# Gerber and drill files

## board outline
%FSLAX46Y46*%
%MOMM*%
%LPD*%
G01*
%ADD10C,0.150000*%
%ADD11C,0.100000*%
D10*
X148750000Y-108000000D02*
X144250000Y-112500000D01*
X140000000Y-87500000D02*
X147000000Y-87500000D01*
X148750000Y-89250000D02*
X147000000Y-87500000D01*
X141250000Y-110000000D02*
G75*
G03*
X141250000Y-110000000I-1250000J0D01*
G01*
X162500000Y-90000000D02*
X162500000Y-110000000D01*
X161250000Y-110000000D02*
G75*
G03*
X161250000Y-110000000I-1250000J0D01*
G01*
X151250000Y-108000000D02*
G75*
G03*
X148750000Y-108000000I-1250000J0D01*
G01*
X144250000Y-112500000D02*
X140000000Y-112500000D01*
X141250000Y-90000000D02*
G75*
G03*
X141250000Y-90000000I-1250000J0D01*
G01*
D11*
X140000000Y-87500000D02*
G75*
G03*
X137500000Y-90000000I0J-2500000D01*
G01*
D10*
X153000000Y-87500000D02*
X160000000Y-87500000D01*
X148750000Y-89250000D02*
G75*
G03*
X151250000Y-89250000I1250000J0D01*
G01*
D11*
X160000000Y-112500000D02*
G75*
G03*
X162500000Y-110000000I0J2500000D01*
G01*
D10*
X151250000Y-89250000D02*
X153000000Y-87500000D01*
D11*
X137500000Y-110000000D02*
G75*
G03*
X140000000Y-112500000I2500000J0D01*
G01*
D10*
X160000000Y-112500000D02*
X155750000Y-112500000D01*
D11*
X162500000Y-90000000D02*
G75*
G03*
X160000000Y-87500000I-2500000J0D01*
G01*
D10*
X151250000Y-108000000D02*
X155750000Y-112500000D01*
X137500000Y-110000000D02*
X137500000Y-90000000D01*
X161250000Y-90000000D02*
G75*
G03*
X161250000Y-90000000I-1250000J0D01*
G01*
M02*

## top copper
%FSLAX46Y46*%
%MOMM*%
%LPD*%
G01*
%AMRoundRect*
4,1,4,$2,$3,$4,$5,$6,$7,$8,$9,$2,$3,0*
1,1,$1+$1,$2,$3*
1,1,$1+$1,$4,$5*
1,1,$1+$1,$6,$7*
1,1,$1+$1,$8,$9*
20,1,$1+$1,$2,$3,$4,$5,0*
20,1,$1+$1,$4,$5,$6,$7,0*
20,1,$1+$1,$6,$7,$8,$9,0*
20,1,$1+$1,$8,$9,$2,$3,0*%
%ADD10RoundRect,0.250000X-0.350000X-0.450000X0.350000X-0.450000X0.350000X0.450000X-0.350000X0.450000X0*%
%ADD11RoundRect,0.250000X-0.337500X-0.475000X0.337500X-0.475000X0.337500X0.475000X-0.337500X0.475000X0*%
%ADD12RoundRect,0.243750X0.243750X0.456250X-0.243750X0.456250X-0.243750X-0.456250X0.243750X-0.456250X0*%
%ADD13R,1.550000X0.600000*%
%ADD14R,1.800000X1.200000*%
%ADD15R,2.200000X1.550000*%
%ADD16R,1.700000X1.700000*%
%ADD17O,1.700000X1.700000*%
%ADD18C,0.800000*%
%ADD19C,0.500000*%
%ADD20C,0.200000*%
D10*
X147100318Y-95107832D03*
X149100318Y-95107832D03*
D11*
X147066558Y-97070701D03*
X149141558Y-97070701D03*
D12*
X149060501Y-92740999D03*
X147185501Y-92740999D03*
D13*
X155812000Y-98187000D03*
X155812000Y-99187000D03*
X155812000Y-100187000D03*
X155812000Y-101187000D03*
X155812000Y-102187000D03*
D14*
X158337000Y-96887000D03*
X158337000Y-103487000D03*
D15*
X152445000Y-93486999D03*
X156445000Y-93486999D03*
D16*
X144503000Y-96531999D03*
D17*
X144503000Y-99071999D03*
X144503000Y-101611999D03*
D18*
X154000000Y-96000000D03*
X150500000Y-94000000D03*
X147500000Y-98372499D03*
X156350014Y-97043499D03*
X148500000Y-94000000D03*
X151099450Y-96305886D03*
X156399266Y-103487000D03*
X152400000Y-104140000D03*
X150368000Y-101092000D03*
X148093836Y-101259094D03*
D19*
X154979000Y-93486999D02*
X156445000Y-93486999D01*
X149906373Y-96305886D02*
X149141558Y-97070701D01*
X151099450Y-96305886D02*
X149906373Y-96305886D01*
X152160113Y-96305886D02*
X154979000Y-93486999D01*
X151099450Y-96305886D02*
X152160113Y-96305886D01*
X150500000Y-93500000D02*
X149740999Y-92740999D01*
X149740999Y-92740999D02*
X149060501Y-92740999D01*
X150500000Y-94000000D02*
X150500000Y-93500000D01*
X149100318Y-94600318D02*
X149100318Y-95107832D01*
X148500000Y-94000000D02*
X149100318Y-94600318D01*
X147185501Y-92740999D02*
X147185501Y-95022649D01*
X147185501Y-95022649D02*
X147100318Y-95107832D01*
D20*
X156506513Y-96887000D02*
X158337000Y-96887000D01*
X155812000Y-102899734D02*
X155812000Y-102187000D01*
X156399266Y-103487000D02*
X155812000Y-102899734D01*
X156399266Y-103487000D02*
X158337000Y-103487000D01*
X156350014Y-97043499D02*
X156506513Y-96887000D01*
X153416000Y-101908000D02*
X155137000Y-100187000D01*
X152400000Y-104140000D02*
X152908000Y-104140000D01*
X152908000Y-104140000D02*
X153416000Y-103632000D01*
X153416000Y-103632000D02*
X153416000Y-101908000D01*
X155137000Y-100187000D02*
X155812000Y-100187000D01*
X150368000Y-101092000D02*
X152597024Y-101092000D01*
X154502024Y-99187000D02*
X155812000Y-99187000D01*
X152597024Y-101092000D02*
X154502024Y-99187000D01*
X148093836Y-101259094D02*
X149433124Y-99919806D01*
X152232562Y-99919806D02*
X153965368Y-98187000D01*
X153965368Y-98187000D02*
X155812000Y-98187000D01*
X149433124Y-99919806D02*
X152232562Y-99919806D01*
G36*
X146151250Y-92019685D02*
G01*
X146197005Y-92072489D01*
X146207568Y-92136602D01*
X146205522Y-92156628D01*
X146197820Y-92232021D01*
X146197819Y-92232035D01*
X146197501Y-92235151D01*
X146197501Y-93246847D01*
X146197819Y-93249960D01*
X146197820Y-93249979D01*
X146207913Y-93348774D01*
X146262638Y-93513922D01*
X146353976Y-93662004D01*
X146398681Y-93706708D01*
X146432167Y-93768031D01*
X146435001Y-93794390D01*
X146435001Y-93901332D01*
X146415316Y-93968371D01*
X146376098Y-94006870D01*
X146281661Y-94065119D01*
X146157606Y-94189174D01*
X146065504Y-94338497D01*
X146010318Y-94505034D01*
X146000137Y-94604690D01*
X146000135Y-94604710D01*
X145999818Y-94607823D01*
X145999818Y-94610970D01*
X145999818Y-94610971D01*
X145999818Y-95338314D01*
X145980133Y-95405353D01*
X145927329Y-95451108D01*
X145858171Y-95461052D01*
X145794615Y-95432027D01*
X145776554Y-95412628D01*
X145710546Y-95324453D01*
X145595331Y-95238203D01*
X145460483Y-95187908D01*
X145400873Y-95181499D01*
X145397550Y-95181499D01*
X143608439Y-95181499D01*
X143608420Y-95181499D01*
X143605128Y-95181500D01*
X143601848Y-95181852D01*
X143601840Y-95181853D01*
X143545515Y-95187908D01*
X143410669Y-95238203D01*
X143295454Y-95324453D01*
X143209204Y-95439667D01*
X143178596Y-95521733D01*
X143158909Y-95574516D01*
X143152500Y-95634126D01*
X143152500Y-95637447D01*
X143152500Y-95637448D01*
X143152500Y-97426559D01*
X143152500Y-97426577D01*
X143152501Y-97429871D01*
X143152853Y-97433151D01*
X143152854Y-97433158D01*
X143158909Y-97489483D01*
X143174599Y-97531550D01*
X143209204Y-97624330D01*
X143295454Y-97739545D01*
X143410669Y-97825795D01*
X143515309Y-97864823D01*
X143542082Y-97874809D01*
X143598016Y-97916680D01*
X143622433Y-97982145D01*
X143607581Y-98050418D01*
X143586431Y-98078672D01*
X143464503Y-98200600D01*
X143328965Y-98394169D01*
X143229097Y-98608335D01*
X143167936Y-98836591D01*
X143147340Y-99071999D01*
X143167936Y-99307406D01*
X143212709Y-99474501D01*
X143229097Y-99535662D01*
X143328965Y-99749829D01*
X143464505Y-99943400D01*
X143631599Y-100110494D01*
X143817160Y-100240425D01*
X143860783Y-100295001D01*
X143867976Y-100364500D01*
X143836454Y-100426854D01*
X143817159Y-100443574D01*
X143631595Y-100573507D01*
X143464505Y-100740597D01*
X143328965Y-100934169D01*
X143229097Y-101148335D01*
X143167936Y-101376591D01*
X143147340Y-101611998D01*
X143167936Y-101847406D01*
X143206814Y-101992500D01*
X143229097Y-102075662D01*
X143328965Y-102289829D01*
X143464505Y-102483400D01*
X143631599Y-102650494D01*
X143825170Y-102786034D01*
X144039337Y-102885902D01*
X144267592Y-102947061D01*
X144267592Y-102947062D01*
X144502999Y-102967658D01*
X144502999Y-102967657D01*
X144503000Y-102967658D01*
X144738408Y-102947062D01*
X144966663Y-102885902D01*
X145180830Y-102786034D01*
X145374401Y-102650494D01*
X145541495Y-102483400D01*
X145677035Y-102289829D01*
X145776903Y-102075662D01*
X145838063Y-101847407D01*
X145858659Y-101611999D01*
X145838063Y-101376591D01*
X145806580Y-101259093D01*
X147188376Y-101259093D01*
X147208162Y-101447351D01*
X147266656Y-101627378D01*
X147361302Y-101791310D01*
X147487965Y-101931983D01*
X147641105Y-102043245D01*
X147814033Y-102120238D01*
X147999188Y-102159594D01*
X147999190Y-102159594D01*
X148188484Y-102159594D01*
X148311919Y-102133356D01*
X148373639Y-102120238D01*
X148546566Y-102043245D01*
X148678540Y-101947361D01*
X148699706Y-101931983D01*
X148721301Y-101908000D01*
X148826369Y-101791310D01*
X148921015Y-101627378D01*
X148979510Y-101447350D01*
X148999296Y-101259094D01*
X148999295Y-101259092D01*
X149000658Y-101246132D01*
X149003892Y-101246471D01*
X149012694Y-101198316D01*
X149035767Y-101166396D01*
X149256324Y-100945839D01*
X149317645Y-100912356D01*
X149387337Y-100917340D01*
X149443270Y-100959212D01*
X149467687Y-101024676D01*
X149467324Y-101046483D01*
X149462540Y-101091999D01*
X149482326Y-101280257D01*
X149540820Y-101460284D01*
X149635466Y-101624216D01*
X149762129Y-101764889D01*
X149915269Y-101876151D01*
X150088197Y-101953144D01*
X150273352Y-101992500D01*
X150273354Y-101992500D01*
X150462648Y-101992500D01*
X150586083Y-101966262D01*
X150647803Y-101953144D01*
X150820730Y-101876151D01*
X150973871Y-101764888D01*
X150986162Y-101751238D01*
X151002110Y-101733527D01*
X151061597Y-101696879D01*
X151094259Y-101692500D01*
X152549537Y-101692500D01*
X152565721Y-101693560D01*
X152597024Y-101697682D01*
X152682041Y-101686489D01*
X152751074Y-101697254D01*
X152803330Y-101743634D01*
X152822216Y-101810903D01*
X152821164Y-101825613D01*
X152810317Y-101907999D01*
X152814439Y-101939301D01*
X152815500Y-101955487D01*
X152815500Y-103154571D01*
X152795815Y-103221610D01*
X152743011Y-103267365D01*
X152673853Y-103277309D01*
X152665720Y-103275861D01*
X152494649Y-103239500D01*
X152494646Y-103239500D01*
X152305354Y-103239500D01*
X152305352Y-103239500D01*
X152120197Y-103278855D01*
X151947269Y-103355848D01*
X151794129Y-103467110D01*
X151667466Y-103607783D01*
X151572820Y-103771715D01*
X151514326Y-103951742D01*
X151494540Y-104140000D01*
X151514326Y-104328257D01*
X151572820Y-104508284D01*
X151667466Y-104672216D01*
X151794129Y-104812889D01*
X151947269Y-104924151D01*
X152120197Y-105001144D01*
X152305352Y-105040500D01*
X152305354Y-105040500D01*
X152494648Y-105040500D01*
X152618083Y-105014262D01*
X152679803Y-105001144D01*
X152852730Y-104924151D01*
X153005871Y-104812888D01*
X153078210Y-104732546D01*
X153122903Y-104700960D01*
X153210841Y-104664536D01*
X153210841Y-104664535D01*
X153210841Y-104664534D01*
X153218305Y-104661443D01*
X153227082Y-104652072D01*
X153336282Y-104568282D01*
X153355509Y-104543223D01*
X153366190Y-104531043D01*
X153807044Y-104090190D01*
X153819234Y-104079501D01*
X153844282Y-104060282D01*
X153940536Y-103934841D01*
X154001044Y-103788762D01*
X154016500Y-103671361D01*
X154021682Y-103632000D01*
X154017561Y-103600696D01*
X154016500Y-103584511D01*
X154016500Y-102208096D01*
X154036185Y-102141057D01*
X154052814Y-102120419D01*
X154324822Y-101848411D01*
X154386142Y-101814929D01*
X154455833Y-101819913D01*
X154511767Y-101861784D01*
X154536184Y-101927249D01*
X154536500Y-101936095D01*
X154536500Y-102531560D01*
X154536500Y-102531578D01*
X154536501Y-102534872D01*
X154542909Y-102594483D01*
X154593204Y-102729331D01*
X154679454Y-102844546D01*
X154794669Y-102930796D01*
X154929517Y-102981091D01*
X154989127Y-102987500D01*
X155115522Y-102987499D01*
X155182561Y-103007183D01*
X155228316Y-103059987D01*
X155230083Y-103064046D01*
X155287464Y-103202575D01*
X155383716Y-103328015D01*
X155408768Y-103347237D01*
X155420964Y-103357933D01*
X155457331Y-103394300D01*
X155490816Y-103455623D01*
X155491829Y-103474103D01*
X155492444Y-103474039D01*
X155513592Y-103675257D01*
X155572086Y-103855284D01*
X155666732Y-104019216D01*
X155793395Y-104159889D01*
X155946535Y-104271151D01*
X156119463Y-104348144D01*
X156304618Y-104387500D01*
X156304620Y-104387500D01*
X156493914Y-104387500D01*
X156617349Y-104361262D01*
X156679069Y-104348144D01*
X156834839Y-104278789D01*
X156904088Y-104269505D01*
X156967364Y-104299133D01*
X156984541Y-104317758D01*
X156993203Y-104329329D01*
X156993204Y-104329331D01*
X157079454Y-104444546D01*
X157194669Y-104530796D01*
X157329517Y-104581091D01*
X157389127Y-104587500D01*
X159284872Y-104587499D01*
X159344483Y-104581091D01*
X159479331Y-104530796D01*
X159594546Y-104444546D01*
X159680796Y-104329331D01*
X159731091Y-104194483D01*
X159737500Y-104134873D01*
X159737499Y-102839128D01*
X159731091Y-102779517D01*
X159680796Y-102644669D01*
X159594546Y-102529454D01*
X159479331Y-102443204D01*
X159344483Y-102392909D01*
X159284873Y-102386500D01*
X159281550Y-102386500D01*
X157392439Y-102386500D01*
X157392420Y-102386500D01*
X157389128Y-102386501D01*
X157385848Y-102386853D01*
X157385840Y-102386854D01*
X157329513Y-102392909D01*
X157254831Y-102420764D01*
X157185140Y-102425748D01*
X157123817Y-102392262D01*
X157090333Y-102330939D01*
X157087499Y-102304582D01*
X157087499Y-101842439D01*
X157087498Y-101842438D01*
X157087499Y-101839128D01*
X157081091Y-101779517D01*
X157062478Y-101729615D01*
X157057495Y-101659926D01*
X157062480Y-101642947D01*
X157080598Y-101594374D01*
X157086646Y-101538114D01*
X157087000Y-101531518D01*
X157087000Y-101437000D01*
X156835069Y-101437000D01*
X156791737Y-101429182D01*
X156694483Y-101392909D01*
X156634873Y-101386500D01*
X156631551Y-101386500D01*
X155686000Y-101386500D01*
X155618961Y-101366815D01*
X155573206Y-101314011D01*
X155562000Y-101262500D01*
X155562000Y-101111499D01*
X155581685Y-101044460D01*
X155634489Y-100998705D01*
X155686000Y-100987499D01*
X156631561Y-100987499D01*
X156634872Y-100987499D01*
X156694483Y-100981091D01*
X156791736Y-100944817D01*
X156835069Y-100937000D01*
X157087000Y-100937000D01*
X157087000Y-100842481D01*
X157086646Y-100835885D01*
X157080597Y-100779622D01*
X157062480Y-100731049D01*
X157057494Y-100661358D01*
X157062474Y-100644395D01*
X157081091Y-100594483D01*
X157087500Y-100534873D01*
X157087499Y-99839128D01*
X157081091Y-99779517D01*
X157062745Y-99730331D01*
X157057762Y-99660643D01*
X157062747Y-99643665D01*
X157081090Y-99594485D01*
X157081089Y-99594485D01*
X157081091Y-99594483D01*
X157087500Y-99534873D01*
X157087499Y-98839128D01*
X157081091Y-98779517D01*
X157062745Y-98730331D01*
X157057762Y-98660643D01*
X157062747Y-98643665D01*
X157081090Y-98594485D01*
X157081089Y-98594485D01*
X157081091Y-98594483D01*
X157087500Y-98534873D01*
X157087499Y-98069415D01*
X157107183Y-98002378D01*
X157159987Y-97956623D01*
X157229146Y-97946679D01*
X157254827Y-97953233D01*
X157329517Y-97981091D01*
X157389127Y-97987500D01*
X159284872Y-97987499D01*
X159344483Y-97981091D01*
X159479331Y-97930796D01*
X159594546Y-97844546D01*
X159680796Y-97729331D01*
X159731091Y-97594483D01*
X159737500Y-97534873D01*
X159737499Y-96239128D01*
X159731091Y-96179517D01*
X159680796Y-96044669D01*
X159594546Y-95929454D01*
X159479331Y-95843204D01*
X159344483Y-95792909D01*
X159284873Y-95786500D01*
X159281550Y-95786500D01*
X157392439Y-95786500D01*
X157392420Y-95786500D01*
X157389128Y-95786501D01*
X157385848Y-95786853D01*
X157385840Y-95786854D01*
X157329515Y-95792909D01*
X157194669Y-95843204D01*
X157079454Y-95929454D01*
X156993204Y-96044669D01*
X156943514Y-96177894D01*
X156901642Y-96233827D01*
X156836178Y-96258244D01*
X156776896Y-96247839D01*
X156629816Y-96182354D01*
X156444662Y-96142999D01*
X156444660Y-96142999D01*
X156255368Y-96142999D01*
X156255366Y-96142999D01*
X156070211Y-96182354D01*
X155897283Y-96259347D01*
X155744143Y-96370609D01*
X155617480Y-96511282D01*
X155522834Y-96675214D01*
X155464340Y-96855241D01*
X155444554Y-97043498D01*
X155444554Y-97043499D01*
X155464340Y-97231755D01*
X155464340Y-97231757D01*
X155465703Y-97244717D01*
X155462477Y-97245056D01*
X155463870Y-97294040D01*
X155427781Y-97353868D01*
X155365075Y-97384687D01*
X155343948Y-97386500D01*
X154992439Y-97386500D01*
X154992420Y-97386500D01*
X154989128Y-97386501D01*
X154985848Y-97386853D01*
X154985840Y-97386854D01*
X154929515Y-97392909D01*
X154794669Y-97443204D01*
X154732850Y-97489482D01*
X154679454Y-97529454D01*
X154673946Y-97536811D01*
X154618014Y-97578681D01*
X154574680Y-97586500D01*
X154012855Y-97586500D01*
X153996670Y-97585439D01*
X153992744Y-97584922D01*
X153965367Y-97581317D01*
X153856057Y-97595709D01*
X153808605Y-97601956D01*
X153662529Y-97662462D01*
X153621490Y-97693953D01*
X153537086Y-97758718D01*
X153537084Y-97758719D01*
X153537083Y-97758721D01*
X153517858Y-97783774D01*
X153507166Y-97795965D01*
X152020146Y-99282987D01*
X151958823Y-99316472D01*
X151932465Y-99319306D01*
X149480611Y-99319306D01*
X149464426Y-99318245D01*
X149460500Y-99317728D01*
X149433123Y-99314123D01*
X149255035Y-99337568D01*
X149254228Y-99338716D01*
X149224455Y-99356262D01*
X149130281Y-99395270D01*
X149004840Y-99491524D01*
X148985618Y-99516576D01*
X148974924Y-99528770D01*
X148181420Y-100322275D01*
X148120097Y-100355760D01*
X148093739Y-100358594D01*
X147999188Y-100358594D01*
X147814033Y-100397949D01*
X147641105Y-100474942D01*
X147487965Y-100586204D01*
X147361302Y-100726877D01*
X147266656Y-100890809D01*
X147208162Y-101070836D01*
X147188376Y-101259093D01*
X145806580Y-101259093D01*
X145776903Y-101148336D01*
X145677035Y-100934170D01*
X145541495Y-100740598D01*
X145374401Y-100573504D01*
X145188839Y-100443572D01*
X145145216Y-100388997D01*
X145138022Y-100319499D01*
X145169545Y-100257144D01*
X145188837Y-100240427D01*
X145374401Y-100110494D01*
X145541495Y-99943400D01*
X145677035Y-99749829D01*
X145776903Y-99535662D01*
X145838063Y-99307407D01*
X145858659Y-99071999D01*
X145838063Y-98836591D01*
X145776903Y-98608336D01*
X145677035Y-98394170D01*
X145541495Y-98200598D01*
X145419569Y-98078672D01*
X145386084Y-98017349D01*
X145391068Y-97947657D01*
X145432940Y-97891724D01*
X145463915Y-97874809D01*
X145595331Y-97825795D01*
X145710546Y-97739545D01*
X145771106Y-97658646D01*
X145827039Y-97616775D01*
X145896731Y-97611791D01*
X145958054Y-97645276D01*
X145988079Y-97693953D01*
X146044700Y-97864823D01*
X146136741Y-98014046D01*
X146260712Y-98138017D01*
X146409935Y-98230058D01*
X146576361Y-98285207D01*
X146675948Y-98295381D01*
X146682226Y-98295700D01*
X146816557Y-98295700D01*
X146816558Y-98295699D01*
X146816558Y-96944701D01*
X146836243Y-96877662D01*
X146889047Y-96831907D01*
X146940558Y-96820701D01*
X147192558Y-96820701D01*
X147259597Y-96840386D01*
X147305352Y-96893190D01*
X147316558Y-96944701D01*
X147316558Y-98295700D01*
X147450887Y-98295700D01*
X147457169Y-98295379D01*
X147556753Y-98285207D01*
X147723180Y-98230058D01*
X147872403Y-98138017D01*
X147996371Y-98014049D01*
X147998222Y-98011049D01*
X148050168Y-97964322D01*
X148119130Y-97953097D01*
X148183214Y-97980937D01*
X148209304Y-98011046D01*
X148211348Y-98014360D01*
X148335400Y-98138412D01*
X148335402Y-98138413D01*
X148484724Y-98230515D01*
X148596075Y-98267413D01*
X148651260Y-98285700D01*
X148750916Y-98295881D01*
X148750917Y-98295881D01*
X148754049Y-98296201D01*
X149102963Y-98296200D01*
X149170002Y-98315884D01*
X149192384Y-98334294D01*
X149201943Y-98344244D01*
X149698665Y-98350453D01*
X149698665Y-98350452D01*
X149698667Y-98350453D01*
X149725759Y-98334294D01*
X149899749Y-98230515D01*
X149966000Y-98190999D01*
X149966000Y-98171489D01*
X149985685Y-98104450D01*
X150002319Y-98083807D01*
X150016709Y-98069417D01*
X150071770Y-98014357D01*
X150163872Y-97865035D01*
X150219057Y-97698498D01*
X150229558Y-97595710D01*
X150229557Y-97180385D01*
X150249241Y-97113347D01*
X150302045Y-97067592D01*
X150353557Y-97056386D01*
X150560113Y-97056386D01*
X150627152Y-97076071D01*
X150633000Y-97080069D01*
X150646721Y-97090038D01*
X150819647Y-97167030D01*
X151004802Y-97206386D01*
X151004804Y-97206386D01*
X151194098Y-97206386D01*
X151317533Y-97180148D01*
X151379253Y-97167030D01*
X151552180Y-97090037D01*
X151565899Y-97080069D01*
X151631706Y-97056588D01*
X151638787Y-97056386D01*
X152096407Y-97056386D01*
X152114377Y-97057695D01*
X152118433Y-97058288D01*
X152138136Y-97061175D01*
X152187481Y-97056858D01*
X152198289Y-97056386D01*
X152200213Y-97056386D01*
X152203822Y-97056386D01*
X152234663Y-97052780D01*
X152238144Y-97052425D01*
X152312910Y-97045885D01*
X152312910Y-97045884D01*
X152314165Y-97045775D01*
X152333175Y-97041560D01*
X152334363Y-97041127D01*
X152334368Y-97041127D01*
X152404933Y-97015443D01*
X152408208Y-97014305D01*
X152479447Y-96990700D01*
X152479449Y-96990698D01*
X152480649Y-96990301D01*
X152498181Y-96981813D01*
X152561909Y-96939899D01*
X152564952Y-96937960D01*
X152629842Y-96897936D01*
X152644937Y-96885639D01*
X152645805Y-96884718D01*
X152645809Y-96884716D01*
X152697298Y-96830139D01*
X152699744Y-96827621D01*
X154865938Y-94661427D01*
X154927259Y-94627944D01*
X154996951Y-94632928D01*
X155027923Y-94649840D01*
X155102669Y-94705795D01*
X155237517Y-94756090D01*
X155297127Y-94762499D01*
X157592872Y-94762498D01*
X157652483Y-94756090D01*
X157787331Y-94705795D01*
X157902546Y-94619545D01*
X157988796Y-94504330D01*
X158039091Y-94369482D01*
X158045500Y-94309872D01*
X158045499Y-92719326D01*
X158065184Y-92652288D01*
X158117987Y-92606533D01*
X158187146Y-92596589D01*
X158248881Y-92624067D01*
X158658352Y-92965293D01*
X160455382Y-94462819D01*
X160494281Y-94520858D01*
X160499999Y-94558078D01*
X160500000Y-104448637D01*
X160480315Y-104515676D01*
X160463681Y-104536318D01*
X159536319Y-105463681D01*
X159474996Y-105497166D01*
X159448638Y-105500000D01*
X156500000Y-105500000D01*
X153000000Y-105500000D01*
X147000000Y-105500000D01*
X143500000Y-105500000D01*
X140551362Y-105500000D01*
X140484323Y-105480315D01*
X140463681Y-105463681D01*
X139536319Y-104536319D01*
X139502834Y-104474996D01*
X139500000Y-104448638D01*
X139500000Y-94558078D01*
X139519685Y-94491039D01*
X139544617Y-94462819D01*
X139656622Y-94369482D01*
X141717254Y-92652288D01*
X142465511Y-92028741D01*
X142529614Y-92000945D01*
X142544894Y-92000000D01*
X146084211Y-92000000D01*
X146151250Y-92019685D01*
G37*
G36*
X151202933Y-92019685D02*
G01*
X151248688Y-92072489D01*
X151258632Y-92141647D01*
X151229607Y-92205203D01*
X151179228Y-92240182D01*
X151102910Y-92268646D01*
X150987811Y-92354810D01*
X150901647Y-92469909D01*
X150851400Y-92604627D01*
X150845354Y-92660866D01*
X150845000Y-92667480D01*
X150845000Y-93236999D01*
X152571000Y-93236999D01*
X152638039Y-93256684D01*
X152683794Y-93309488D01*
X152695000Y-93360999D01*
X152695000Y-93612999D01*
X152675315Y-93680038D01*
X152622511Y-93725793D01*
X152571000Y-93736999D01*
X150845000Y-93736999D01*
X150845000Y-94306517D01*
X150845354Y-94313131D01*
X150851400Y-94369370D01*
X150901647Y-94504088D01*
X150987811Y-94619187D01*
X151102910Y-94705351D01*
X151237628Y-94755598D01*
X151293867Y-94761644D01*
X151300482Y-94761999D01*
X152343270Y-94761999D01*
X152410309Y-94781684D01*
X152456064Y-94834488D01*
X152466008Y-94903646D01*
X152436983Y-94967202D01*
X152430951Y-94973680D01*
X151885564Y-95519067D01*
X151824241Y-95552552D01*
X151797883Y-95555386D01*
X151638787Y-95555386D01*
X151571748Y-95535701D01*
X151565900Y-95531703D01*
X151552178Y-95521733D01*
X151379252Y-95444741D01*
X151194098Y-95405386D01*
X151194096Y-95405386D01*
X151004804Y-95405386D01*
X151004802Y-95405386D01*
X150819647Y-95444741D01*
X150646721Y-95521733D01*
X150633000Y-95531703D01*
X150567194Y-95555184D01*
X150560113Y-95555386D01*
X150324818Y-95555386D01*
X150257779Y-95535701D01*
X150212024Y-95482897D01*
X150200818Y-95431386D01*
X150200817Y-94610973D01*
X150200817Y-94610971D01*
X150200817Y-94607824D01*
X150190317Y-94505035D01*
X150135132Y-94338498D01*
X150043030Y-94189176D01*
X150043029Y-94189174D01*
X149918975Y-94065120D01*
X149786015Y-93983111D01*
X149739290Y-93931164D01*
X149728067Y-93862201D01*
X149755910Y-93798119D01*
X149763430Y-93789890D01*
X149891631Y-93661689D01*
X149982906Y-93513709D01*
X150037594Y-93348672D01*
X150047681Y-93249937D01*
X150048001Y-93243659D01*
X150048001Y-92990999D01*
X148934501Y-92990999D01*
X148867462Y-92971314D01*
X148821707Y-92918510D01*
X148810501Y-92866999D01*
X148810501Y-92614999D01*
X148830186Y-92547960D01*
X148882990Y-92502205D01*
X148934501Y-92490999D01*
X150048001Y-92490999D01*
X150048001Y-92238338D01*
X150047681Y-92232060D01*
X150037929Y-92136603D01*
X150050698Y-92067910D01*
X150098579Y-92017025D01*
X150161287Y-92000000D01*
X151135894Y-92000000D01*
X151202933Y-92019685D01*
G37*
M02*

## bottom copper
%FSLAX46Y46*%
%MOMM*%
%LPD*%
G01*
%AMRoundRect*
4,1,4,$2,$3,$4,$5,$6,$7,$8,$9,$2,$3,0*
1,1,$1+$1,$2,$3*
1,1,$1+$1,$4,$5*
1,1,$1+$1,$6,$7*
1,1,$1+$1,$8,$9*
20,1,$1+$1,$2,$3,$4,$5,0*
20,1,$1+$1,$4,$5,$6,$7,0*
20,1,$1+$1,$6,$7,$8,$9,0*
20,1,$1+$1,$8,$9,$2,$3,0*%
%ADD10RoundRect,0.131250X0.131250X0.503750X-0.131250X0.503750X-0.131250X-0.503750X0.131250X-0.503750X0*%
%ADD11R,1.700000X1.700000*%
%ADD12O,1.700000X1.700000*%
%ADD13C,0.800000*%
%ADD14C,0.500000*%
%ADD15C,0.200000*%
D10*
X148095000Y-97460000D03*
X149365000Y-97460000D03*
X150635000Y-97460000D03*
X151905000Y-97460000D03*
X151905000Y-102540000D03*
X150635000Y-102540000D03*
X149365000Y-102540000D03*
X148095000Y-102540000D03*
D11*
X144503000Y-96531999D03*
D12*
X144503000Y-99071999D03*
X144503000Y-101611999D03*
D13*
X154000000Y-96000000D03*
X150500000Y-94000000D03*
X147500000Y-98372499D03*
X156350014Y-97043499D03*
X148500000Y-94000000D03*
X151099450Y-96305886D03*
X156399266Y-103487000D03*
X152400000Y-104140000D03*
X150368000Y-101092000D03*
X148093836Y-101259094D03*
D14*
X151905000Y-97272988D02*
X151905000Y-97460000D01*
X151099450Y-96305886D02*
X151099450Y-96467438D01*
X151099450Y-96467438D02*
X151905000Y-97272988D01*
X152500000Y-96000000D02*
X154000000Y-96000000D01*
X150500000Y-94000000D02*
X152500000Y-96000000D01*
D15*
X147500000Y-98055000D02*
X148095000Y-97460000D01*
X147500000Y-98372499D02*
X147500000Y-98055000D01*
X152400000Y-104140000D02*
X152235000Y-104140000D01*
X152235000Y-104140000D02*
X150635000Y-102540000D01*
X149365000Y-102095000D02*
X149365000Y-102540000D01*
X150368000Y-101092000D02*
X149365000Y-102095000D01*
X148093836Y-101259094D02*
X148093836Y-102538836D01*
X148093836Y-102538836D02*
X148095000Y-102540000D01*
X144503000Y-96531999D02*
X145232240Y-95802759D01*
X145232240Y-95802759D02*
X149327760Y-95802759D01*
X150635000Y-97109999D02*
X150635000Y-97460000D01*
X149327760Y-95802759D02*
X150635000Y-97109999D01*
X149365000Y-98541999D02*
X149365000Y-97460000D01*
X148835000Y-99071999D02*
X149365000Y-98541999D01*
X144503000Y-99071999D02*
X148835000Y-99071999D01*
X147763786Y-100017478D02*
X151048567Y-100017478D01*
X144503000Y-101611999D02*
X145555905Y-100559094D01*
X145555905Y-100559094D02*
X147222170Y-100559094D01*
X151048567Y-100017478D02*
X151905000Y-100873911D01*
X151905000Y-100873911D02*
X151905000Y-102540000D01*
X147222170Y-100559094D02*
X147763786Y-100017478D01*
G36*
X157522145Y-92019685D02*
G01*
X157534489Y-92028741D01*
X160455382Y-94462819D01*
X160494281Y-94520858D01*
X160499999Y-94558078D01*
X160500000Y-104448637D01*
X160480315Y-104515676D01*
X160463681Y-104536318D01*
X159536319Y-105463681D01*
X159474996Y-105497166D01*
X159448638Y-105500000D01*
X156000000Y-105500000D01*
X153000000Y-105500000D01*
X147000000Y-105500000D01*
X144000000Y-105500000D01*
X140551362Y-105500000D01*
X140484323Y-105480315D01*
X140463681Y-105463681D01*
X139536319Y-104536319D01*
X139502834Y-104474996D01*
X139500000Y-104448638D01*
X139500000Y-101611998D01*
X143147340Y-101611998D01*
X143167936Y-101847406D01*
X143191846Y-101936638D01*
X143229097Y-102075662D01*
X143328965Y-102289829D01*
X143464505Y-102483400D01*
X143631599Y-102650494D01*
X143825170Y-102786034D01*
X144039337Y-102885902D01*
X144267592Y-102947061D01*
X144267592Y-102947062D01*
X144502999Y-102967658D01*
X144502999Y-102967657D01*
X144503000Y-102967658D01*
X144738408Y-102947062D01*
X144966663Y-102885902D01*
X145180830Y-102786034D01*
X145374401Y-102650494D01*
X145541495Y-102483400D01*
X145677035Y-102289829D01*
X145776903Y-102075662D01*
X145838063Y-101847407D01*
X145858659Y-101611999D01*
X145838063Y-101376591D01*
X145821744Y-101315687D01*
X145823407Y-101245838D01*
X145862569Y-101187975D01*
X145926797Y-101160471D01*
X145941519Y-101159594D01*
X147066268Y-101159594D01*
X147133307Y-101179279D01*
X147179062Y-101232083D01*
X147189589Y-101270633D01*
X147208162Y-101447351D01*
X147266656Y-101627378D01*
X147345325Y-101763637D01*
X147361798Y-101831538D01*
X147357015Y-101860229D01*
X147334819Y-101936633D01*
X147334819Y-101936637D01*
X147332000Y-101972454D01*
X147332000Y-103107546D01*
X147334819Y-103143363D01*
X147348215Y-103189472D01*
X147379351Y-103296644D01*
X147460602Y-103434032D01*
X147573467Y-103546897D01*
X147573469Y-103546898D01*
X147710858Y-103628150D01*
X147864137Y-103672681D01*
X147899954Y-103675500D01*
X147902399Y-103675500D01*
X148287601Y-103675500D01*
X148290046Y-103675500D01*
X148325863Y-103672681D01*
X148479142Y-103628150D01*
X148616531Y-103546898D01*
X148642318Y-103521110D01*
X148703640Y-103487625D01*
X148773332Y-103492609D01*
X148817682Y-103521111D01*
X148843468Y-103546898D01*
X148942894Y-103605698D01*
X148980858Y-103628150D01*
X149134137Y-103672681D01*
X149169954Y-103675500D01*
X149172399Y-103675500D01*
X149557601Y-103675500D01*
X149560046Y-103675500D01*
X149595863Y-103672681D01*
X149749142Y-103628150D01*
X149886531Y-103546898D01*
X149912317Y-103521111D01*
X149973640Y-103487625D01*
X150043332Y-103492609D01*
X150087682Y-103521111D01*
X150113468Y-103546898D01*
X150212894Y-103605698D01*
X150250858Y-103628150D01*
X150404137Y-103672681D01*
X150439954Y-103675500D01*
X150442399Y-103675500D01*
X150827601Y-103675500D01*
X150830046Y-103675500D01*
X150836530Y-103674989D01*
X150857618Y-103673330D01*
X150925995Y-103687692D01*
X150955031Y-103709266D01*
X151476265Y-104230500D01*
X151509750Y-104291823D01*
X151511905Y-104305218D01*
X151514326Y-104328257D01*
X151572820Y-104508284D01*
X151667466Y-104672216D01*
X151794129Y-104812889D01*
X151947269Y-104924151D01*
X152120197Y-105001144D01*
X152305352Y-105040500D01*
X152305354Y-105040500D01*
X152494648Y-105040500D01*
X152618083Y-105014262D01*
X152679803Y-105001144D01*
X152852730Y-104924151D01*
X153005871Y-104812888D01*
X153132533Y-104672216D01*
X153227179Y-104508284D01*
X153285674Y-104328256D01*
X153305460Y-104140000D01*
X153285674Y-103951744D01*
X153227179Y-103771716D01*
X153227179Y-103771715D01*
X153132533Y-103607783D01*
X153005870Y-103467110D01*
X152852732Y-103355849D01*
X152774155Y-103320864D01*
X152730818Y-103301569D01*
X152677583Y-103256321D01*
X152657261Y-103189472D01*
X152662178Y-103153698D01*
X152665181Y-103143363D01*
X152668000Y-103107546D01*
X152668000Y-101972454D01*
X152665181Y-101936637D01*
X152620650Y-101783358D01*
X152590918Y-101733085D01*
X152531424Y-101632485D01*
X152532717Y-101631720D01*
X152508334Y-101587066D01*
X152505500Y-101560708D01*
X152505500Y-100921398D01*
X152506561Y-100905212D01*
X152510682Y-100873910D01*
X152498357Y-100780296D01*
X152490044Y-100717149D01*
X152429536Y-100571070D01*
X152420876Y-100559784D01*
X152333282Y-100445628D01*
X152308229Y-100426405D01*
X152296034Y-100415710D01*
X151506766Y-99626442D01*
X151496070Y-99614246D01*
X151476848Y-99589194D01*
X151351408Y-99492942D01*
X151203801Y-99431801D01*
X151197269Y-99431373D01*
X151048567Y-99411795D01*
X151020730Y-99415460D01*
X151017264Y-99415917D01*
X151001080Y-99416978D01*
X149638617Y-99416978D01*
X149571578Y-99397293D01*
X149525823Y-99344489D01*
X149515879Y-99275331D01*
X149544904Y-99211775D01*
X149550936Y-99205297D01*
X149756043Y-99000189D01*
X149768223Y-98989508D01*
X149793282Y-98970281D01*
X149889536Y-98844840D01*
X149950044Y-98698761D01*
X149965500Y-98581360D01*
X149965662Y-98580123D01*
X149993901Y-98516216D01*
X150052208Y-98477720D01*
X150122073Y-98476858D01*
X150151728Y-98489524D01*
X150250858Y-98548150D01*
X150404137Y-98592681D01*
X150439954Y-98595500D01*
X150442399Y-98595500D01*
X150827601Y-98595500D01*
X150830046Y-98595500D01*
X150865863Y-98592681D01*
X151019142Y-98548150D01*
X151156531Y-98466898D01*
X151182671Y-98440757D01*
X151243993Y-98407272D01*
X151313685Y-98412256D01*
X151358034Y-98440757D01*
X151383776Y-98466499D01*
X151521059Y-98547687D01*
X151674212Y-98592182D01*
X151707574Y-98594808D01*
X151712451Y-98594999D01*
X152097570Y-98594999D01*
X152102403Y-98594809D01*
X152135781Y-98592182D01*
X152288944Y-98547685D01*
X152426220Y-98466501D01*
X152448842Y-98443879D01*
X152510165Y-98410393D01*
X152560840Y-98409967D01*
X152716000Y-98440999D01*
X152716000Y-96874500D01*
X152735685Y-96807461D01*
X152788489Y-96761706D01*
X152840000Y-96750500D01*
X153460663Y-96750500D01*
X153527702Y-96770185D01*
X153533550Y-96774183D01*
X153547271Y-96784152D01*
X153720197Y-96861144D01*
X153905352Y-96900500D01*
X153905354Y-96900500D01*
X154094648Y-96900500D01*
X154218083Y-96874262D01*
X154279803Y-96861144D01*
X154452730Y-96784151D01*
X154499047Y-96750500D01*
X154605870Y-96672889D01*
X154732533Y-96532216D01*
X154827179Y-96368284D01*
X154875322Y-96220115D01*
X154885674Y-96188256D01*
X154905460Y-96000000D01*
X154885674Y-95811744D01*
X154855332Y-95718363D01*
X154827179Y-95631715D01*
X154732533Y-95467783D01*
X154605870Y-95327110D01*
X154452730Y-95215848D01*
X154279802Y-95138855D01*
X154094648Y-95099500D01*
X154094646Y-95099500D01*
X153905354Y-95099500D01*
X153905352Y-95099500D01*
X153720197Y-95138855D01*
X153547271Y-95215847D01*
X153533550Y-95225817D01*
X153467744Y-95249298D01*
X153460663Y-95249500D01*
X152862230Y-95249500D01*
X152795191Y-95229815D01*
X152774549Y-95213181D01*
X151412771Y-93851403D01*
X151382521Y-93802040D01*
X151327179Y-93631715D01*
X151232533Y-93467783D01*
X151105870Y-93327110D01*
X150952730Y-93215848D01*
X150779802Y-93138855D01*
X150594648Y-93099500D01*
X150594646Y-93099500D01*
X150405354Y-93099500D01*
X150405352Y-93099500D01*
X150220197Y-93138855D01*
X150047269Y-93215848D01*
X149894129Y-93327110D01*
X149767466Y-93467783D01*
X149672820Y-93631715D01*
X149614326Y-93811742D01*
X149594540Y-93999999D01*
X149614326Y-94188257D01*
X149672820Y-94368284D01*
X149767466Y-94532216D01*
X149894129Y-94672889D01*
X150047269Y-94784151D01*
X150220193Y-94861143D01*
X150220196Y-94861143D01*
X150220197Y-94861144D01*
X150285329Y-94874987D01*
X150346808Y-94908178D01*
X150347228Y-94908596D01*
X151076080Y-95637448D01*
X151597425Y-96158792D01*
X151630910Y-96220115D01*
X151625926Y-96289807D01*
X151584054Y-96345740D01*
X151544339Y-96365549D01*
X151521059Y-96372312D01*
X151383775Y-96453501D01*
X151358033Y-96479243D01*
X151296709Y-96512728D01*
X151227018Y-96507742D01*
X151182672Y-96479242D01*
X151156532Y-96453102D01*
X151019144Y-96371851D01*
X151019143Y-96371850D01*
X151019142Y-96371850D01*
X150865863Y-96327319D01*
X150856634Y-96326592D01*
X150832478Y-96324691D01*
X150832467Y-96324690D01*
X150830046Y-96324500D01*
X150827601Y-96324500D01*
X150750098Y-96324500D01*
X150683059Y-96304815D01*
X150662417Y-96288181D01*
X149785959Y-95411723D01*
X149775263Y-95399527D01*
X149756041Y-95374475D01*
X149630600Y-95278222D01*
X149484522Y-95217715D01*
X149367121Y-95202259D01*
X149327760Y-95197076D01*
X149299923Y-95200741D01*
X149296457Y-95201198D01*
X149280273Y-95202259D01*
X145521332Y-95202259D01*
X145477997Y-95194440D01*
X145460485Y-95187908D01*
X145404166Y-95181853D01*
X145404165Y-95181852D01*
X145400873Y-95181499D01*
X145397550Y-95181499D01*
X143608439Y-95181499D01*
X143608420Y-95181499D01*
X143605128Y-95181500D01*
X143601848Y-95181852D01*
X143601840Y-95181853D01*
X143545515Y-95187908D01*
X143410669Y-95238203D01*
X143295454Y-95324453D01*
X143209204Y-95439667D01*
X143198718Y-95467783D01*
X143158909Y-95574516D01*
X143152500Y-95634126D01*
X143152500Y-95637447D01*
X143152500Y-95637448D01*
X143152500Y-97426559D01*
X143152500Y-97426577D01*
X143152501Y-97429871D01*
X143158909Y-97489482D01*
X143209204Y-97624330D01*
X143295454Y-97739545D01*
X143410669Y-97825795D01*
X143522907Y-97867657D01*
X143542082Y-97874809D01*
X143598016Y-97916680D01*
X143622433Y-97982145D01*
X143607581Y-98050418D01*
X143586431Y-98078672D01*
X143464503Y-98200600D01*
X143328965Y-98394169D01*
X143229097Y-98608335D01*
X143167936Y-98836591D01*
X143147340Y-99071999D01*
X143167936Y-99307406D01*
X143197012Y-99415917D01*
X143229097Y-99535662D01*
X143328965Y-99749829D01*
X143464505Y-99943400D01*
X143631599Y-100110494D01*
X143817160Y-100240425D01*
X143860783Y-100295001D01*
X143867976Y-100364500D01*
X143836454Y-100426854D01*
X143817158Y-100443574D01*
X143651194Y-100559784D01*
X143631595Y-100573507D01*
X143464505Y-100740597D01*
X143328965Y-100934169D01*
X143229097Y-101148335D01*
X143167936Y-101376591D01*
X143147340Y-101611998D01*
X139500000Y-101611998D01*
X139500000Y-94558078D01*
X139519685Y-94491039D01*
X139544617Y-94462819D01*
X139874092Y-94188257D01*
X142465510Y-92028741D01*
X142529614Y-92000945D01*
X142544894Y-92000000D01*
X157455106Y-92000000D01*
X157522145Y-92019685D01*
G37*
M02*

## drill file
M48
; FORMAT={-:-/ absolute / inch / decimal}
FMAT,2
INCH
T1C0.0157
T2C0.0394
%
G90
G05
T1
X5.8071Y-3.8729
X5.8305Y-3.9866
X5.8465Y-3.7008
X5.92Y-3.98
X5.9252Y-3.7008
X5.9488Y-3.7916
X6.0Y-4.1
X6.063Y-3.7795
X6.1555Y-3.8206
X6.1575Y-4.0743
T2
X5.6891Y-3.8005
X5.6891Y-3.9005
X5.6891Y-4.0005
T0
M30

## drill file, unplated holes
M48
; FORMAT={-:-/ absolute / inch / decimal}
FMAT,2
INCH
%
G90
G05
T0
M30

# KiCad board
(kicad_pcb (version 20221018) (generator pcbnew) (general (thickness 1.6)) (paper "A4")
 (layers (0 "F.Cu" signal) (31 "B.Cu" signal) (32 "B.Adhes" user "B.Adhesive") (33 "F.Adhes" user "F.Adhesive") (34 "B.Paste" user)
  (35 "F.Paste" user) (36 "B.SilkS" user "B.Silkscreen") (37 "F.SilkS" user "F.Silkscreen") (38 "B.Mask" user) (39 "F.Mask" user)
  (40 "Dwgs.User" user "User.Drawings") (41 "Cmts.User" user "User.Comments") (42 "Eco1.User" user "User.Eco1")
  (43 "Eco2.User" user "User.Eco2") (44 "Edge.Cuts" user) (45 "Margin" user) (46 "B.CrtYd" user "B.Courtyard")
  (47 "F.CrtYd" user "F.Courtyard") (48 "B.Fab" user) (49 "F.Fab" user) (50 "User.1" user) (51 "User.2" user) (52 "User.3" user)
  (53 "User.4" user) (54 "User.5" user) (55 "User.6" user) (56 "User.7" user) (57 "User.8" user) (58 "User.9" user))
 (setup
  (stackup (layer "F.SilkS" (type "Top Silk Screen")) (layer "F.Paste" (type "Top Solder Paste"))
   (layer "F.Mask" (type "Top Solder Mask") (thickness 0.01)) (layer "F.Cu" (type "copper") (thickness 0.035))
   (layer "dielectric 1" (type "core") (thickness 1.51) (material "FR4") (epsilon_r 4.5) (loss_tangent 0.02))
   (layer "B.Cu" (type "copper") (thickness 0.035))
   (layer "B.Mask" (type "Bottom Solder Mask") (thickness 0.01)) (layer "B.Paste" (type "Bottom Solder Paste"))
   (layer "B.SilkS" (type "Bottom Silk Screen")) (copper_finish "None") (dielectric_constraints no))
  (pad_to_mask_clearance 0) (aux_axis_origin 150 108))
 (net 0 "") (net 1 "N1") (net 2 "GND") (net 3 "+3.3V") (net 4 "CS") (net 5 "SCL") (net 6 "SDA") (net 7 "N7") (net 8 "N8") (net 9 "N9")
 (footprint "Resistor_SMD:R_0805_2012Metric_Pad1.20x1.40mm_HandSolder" (layer "F.Cu") (at 148.100318 95.107832)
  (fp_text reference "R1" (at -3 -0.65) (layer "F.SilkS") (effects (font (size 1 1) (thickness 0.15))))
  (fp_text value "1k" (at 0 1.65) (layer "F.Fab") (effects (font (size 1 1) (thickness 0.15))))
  (pad "1" smd roundrect (at -1 0) (size 1.2 1.4) (layers "F.Cu" "F.Paste" "F.Mask") (roundrect_rratio 0.208333) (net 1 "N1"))
  (pad "2" smd roundrect (at 1 0) (size 1.2 1.4) (layers "F.Cu" "F.Paste" "F.Mask") (roundrect_rratio 0.208333) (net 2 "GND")))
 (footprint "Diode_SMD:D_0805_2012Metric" (layer "F.Cu") (at 148.123001 92.740999 180)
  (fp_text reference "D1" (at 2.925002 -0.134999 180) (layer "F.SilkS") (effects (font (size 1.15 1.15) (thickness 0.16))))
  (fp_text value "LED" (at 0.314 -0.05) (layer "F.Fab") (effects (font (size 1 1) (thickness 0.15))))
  (pad "1" smd roundrect (at -0.9375 0 180) (size 0.975 1.4) (layers "F.Cu" "F.Paste" "F.Mask") (roundrect_rratio 0.25) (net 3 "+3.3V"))
  (pad "2" smd roundrect (at 0.9375 0 180) (size 0.975 1.4) (layers "F.Cu" "F.Paste" "F.Mask") (roundrect_rratio 0.25) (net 1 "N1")))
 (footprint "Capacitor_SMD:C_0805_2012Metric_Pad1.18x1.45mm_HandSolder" (layer "F.Cu") (at 148.104058 97.070701)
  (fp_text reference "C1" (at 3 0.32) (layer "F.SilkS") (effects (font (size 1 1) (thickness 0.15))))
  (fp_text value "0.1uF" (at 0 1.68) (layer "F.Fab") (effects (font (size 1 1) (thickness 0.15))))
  (pad "1" smd roundrect (at -1.0375 0) (size 1.175 1.45) (layers "F.Cu" "F.Paste" "F.Mask") (roundrect_rratio 0.212766) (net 3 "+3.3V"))
  (pad "2" smd roundrect (at 1.0375 0) (size 1.175 1.45) (layers "F.Cu" "F.Paste" "F.Mask") (roundrect_rratio 0.212766) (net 2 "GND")))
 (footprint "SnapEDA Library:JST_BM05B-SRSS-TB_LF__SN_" (layer "F.Cu") (at 158.337 100.187 -90)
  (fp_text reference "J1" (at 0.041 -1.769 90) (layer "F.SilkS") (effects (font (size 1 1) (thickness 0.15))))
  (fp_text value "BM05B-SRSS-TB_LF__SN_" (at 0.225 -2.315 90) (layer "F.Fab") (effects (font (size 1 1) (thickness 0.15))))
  (pad "1" smd rect (at -2 2.525 270) (size 0.6 1.55) (layers "F.Cu" "F.Paste" "F.Mask") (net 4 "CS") (solder_mask_margin 0.102))
  (pad "2" smd rect (at -1 2.525 270) (size 0.6 1.55) (layers "F.Cu" "F.Paste" "F.Mask") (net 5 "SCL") (solder_mask_margin 0.102))
  (pad "3" smd rect (at 0 2.525 270) (size 0.6 1.55) (layers "F.Cu" "F.Paste" "F.Mask") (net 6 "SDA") (solder_mask_margin 0.102))
  (pad "4" smd rect (at 1 2.525 270) (size 0.6 1.55) (layers "F.Cu" "F.Paste" "F.Mask") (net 3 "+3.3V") (solder_mask_margin 0.102))
  (pad "5" smd rect (at 2 2.525 270) (size 0.6 1.55) (layers "F.Cu" "F.Paste" "F.Mask") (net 2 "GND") (solder_mask_margin 0.102))
  (pad "S1" smd rect (at -3.3 0 270) (size 1.2 1.8) (layers "F.Cu" "F.Paste" "F.Mask") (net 2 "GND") (solder_mask_margin 0.102))
  (pad "S2" smd rect (at 3.3 0 270) (size 1.2 1.8) (layers "F.Cu" "F.Paste" "F.Mask") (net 2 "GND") (solder_mask_margin 0.102)))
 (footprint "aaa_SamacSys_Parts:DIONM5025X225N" (layer "F.Cu") (at 154.445 93.486999)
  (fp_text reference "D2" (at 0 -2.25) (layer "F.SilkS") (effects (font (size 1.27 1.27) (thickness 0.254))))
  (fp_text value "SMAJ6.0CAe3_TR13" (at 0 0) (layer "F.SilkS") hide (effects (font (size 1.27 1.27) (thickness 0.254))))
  (pad "1" smd rect (at -2 0 90) (size 1.55 2.2) (layers "F.Cu" "F.Paste" "F.Mask") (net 3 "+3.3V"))
  (pad "2" smd rect (at 2 0 90) (size 1.55 2.2) (layers "F.Cu" "F.Paste" "F.Mask") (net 2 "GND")))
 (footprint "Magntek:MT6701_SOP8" (layer "B.Cu") (at 150 100)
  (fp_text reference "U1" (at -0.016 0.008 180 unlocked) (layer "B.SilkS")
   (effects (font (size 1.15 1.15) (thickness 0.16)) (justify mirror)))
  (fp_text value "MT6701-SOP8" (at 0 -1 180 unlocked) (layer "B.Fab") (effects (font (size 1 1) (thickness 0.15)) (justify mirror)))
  (pad "1" smd roundrect (at -1.905 -2.54 180) (size 0.525 1.27) (layers "B.Cu" "B.Paste" "B.Mask") (roundrect_rratio 0.25) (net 3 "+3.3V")
   (thermal_bridge_angle 45))
  (pad "2" smd roundrect (at -0.635 -2.54 180) (size 0.525 1.27) (layers "B.Cu" "B.Paste" "B.Mask") (roundrect_rratio 0.25) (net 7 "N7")
   (thermal_bridge_angle 45))
  (pad "3" smd roundrect (at 0.635 -2.54 180) (size 0.525 1.27) (layers "B.Cu" "B.Paste" "B.Mask") (roundrect_rratio 0.25) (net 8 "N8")
   (thermal_bridge_angle 45))
  (pad "4" smd roundrect (at 1.905 -2.54 180) (size 0.525 1.27) (layers "B.Cu" "B.Paste" "B.Mask") (roundrect_rratio 0.25) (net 2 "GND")
   (thermal_bridge_angle 45))
  (pad "5" smd roundrect (at 1.905 2.54 180) (size 0.525 1.27) (layers "B.Cu" "B.Paste" "B.Mask") (roundrect_rratio 0.25) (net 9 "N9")
   (thermal_bridge_angle 45))
  (pad "6" smd roundrect (at 0.635 2.54 180) (size 0.525 1.27) (layers "B.Cu" "B.Paste" "B.Mask") (roundrect_rratio 0.25) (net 6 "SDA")
   (thermal_bridge_angle 45))
  (pad "7" smd roundrect (at -0.635 2.54 180) (size 0.525 1.27) (layers "B.Cu" "B.Paste" "B.Mask") (roundrect_rratio 0.25) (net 5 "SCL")
   (thermal_bridge_angle 45))
  (pad "8" smd roundrect (at -1.905 2.54 180) (size 0.525 1.27) (layers "B.Cu" "B.Paste" "B.Mask") (roundrect_rratio 0.25) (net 4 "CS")
   (thermal_bridge_angle 45)))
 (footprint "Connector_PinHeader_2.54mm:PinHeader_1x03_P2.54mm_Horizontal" (layer "B.Cu") (at 144.503 96.531999 180)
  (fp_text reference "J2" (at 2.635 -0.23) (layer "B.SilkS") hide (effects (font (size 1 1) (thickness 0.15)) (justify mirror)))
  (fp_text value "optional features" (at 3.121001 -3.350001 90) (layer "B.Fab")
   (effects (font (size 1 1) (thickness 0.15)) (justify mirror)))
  (pad "1" thru_hole rect (at 0 0 180) (size 1.7 1.7) (drill 1) (layers "*.Cu" "*.Mask") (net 8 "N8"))
  (pad "2" thru_hole oval (at 0 -2.54 180) (size 1.7 1.7) (drill 1) (layers "*.Cu" "*.Mask") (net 7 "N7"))
  (pad "3" thru_hole oval (at 0 -5.08 180) (size 1.7 1.7) (drill 1) (layers "*.Cu" "*.Mask") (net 9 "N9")))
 (gr_line (start 148.75 108) (end 144.25 112.5) (stroke (width 0.15) (type default)) (layer "Edge.Cuts"))
 (gr_line (start 140 87.5) (end 147 87.5) (stroke (width 0.15) (type default)) (layer "Edge.Cuts"))
 (gr_line (start 148.75 89.25) (end 147 87.5) (stroke (width 0.15) (type default)) (layer "Edge.Cuts"))
 (gr_circle (center 140 110) (end 141.25 110) (stroke (width 0.15) (type default)) (fill none) (layer "Edge.Cuts"))
 (gr_line (start 162.5 90) (end 162.5 110) (stroke (width 0.15) (type default)) (layer "Edge.Cuts"))
 (gr_circle (center 160 110) (end 161.25 110) (stroke (width 0.15) (type default)) (fill none) (layer "Edge.Cuts"))
 (gr_arc (start 148.75 108) (mid 150 106.75) (end 151.25 108) (stroke (width 0.15) (type default)) (layer "Edge.Cuts"))
 (gr_line (start 144.25 112.5) (end 140 112.5) (stroke (width 0.15) (type default)) (layer "Edge.Cuts"))
 (gr_circle (center 140 90) (end 141.25 90) (stroke (width 0.15) (type default)) (fill none) (layer "Edge.Cuts"))
 (gr_arc (start 137.5 90) (mid 138.232233 88.232233) (end 140 87.5) (stroke (width 0.1) (type default)) (layer "Edge.Cuts"))
 (gr_line (start 153 87.5) (end 160 87.5) (stroke (width 0.15) (type default)) (layer "Edge.Cuts"))
 (gr_arc (start 151.25 89.25) (mid 150 90.5) (end 148.75 89.25) (stroke (width 0.15) (type default)) (layer "Edge.Cuts"))
 (gr_arc (start 162.5 110) (mid 161.767767 111.767767) (end 160 112.5) (stroke (width 0.1) (type default)) (layer "Edge.Cuts"))
 (gr_line (start 151.25 89.25) (end 153 87.5) (stroke (width 0.15) (type default)) (layer "Edge.Cuts"))
 (gr_arc (start 140 112.5) (mid 138.232233 111.767767) (end 137.5 110) (stroke (width 0.1) (type default)) (layer "Edge.Cuts"))
 (gr_line (start 160 112.5) (end 155.75 112.5) (stroke (width 0.15) (type default)) (layer "Edge.Cuts"))
 (gr_arc (start 160 87.5) (mid 161.767767 88.232233) (end 162.5 90) (stroke (width 0.1) (type default)) (layer "Edge.Cuts"))
 (gr_line (start 151.25 108) (end 155.75 112.5) (stroke (width 0.15) (type default)) (layer "Edge.Cuts"))
 (gr_line (start 137.5 110) (end 137.5 90) (stroke (width 0.15) (type default)) (layer "Edge.Cuts"))
 (gr_circle (center 160 90) (end 161.25 90) (stroke (width 0.15) (type default)) (fill none) (layer "Edge.Cuts"))
 (segment (start 150.5 93.5) (end 149.740999 92.740999) (width 0.5) (layer "F.Cu") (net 3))
 (segment (start 149.740999 92.740999) (end 149.060501 92.740999) (width 0.5) (layer "F.Cu") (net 3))
 (segment (start 150.5 94) (end 150.5 93.5) (width 0.5) (layer "F.Cu") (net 3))
 (via (at 150.5 94) (size 0.8) (drill 0.4) (layers "F.Cu" "B.Cu") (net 3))
 (via (at 147.5 98.372499) (size 0.8) (drill 0.4) (layers "F.Cu" "B.Cu") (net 3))
 (via (at 154 96) (size 0.8) (drill 0.4) (layers "F.Cu" "B.Cu") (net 3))
 (segment (start 147.5 98.055) (end 148.095 97.46) (width 0.2) (layer "B.Cu") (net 3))
 (segment (start 150.5 94) (end 152.5 96) (width 0.5) (layer "B.Cu") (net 3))
 (segment (start 147.5 98.372499) (end 147.5 98.055) (width 0.2) (layer "B.Cu") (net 3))
 (segment (start 152.5 96) (end 154 96) (width 0.5) (layer "B.Cu") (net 3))
 (segment (start 148.5 94) (end 149.100318 94.600318) (width 0.5) (layer "F.Cu") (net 2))
 (segment (start 156.506513 96.887) (end 158.337 96.887) (width 0.2) (layer "F.Cu") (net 2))
 (segment (start 155.812 102.899734) (end 155.812 102.187) (width 0.2) (layer "F.Cu") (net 2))
 (segment (start 156.399266 103.487) (end 155.812 102.899734) (width 0.2) (layer "F.Cu") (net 2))
 (segment (start 149.100318 94.600318) (end 149.100318 95.107832) (width 0.5) (layer "F.Cu") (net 2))
 (segment (start 151.09945 96.305886) (end 149.906373 96.305886) (width 0.5) (layer "F.Cu") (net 2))
 (segment (start 151.09945 96.305886) (end 152.160113 96.305886) (width 0.5) (layer "F.Cu") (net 2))
 (segment (start 149.906373 96.305886) (end 149.141558 97.070701) (width 0.5) (layer "F.Cu") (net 2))
 (segment (start 156.399266 103.487) (end 158.337 103.487) (width 0.2) (layer "F.Cu") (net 2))
 (segment (start 152.160113 96.305886) (end 154.979 93.486999) (width 0.5) (layer "F.Cu") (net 2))
 (segment (start 156.350014 97.043499) (end 156.506513 96.887) (width 0.2) (layer "F.Cu") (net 2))
 (segment (start 154.979 93.486999) (end 156.445 93.486999) (width 0.5) (layer "F.Cu") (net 2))
 (via (at 156.350014 97.043499) (size 0.8) (drill 0.4) (layers "F.Cu" "B.Cu") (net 2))
 (via (at 148.5 94) (size 0.8) (drill 0.4) (layers "F.Cu" "B.Cu") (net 2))
 (via (at 151.09945 96.305886) (size 0.8) (drill 0.4) (layers "F.Cu" "B.Cu") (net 2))
 (via (at 156.399266 103.487) (size 0.8) (drill 0.4) (layers "F.Cu" "B.Cu") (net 2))
 (segment (start 151.905 97.272988) (end 151.905 97.46) (width 0.5) (layer "B.Cu") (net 2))
 (segment (start 151.09945 96.467438) (end 151.905 97.272988) (width 0.5) (layer "B.Cu") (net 2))
 (segment (start 151.09945 96.305886) (end 151.09945 96.467438) (width 0.5) (layer "B.Cu") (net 2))
 (segment (start 147.185501 95.022649) (end 147.100318 95.107832) (width 0.5) (layer "F.Cu") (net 1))
 (segment (start 147.185501 92.740999) (end 147.185501 95.022649) (width 0.5) (layer "F.Cu") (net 1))
 (segment (start 153.416 101.908) (end 155.137 100.187) (width 0.2) (layer "F.Cu") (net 6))
 (segment (start 152.4 104.14) (end 152.908 104.14) (width 0.2) (layer "F.Cu") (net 6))
 (segment (start 152.908 104.14) (end 153.416 103.632) (width 0.2) (layer "F.Cu") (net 6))
 (segment (start 153.416 103.632) (end 153.416 101.908) (width 0.2) (layer "F.Cu") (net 6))
 (segment (start 155.137 100.187) (end 155.812 100.187) (width 0.2) (layer "F.Cu") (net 6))
 (via (at 152.4 104.14) (size 0.8) (drill 0.4) (layers "F.Cu" "B.Cu") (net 6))
 (segment (start 152.4 104.14) (end 152.235 104.14) (width 0.2) (layer "B.Cu") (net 6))
 (segment (start 152.235 104.14) (end 150.635 102.54) (width 0.2) (layer "B.Cu") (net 6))
 (segment (start 150.368 101.092) (end 152.597024 101.092) (width 0.2) (layer "F.Cu") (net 5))
 (segment (start 154.502024 99.187) (end 155.812 99.187) (width 0.2) (layer "F.Cu") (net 5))
 (segment (start 152.597024 101.092) (end 154.502024 99.187) (width 0.2) (layer "F.Cu") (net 5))
 (via (at 150.368 101.092) (size 0.8) (drill 0.4) (layers "F.Cu" "B.Cu") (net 5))
 (segment (start 149.365 102.095) (end 149.365 102.54) (width 0.2) (layer "B.Cu") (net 5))
 (segment (start 150.368 101.092) (end 149.365 102.095) (width 0.2) (layer "B.Cu") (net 5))
 (segment (start 148.093836 101.259094) (end 149.433124 99.919806) (width 0.2) (layer "F.Cu") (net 4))
 (segment (start 152.232562 99.919806) (end 153.965368 98.187) (width 0.2) (layer "F.Cu") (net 4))
 (segment (start 153.965368 98.187) (end 155.812 98.187) (width 0.2) (layer "F.Cu") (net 4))
 (segment (start 149.433124 99.919806) (end 152.232562 99.919806) (width 0.2) (layer "F.Cu") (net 4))
 (via (at 148.093836 101.259094) (size 0.8) (drill 0.4) (layers "F.Cu" "B.Cu") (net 4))
 (segment (start 148.093836 101.259094) (end 148.093836 102.538836) (width 0.2) (layer "B.Cu") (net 4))
 (segment (start 148.093836 102.538836) (end 148.095 102.54) (width 0.2) (layer "B.Cu") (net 4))
 (segment (start 144.503 96.531999) (end 145.23224 95.802759) (width 0.2) (layer "B.Cu") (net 8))
 (segment (start 145.23224 95.802759) (end 149.32776 95.802759) (width 0.2) (layer "B.Cu") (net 8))
 (segment (start 150.635 97.109999) (end 150.635 97.46) (width 0.2) (layer "B.Cu") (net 8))
 (segment (start 149.32776 95.802759) (end 150.635 97.109999) (width 0.2) (layer "B.Cu") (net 8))
 (segment (start 149.365 98.541999) (end 149.365 97.46) (width 0.2) (layer "B.Cu") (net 7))
 (segment (start 148.835 99.071999) (end 149.365 98.541999) (width 0.2) (layer "B.Cu") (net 7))
 (segment (start 144.503 99.071999) (end 148.835 99.071999) (width 0.2) (layer "B.Cu") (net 7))
 (segment (start 147.763786 100.017478) (end 151.048567 100.017478) (width 0.2) (layer "B.Cu") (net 9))
 (segment (start 144.503 101.611999) (end 145.555905 100.559094) (width 0.2) (layer "B.Cu") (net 9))
 (segment (start 145.555905 100.559094) (end 147.22217 100.559094) (width 0.2) (layer "B.Cu") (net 9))
 (segment (start 151.048567 100.017478) (end 151.905 100.873911) (width 0.2) (layer "B.Cu") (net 9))
 (segment (start 151.905 100.873911) (end 151.905 102.54) (width 0.2) (layer "B.Cu") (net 9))
 (segment (start 147.22217 100.559094) (end 147.763786 100.017478) (width 0.2) (layer "B.Cu") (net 9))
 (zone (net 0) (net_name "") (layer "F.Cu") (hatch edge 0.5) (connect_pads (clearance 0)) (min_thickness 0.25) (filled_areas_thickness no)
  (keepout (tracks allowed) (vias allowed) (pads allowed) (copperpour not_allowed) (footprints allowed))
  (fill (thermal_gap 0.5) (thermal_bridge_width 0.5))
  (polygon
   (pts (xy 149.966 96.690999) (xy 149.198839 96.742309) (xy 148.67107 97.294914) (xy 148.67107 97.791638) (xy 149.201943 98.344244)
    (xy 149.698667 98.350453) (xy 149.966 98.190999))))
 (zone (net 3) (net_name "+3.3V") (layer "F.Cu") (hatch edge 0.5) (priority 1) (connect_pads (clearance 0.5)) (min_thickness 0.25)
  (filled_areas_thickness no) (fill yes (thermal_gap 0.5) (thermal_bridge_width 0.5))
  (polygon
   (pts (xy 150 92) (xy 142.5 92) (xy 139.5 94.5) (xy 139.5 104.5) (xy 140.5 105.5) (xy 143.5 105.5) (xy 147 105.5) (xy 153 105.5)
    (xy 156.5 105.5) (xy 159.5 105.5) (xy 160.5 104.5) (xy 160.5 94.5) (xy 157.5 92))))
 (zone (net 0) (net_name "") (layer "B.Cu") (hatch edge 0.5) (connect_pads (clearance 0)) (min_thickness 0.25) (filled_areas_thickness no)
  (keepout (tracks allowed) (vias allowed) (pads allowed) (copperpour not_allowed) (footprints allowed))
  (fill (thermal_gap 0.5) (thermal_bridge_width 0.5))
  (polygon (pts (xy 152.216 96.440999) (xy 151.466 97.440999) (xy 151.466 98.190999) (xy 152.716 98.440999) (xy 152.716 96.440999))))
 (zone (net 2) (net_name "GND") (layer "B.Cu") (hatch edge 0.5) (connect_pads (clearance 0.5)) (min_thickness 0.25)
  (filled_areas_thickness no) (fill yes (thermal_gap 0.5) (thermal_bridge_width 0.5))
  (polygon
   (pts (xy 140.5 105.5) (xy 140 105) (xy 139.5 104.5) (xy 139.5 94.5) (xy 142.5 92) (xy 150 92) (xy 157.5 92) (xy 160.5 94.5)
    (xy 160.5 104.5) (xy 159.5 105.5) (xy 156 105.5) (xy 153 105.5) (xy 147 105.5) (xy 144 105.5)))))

